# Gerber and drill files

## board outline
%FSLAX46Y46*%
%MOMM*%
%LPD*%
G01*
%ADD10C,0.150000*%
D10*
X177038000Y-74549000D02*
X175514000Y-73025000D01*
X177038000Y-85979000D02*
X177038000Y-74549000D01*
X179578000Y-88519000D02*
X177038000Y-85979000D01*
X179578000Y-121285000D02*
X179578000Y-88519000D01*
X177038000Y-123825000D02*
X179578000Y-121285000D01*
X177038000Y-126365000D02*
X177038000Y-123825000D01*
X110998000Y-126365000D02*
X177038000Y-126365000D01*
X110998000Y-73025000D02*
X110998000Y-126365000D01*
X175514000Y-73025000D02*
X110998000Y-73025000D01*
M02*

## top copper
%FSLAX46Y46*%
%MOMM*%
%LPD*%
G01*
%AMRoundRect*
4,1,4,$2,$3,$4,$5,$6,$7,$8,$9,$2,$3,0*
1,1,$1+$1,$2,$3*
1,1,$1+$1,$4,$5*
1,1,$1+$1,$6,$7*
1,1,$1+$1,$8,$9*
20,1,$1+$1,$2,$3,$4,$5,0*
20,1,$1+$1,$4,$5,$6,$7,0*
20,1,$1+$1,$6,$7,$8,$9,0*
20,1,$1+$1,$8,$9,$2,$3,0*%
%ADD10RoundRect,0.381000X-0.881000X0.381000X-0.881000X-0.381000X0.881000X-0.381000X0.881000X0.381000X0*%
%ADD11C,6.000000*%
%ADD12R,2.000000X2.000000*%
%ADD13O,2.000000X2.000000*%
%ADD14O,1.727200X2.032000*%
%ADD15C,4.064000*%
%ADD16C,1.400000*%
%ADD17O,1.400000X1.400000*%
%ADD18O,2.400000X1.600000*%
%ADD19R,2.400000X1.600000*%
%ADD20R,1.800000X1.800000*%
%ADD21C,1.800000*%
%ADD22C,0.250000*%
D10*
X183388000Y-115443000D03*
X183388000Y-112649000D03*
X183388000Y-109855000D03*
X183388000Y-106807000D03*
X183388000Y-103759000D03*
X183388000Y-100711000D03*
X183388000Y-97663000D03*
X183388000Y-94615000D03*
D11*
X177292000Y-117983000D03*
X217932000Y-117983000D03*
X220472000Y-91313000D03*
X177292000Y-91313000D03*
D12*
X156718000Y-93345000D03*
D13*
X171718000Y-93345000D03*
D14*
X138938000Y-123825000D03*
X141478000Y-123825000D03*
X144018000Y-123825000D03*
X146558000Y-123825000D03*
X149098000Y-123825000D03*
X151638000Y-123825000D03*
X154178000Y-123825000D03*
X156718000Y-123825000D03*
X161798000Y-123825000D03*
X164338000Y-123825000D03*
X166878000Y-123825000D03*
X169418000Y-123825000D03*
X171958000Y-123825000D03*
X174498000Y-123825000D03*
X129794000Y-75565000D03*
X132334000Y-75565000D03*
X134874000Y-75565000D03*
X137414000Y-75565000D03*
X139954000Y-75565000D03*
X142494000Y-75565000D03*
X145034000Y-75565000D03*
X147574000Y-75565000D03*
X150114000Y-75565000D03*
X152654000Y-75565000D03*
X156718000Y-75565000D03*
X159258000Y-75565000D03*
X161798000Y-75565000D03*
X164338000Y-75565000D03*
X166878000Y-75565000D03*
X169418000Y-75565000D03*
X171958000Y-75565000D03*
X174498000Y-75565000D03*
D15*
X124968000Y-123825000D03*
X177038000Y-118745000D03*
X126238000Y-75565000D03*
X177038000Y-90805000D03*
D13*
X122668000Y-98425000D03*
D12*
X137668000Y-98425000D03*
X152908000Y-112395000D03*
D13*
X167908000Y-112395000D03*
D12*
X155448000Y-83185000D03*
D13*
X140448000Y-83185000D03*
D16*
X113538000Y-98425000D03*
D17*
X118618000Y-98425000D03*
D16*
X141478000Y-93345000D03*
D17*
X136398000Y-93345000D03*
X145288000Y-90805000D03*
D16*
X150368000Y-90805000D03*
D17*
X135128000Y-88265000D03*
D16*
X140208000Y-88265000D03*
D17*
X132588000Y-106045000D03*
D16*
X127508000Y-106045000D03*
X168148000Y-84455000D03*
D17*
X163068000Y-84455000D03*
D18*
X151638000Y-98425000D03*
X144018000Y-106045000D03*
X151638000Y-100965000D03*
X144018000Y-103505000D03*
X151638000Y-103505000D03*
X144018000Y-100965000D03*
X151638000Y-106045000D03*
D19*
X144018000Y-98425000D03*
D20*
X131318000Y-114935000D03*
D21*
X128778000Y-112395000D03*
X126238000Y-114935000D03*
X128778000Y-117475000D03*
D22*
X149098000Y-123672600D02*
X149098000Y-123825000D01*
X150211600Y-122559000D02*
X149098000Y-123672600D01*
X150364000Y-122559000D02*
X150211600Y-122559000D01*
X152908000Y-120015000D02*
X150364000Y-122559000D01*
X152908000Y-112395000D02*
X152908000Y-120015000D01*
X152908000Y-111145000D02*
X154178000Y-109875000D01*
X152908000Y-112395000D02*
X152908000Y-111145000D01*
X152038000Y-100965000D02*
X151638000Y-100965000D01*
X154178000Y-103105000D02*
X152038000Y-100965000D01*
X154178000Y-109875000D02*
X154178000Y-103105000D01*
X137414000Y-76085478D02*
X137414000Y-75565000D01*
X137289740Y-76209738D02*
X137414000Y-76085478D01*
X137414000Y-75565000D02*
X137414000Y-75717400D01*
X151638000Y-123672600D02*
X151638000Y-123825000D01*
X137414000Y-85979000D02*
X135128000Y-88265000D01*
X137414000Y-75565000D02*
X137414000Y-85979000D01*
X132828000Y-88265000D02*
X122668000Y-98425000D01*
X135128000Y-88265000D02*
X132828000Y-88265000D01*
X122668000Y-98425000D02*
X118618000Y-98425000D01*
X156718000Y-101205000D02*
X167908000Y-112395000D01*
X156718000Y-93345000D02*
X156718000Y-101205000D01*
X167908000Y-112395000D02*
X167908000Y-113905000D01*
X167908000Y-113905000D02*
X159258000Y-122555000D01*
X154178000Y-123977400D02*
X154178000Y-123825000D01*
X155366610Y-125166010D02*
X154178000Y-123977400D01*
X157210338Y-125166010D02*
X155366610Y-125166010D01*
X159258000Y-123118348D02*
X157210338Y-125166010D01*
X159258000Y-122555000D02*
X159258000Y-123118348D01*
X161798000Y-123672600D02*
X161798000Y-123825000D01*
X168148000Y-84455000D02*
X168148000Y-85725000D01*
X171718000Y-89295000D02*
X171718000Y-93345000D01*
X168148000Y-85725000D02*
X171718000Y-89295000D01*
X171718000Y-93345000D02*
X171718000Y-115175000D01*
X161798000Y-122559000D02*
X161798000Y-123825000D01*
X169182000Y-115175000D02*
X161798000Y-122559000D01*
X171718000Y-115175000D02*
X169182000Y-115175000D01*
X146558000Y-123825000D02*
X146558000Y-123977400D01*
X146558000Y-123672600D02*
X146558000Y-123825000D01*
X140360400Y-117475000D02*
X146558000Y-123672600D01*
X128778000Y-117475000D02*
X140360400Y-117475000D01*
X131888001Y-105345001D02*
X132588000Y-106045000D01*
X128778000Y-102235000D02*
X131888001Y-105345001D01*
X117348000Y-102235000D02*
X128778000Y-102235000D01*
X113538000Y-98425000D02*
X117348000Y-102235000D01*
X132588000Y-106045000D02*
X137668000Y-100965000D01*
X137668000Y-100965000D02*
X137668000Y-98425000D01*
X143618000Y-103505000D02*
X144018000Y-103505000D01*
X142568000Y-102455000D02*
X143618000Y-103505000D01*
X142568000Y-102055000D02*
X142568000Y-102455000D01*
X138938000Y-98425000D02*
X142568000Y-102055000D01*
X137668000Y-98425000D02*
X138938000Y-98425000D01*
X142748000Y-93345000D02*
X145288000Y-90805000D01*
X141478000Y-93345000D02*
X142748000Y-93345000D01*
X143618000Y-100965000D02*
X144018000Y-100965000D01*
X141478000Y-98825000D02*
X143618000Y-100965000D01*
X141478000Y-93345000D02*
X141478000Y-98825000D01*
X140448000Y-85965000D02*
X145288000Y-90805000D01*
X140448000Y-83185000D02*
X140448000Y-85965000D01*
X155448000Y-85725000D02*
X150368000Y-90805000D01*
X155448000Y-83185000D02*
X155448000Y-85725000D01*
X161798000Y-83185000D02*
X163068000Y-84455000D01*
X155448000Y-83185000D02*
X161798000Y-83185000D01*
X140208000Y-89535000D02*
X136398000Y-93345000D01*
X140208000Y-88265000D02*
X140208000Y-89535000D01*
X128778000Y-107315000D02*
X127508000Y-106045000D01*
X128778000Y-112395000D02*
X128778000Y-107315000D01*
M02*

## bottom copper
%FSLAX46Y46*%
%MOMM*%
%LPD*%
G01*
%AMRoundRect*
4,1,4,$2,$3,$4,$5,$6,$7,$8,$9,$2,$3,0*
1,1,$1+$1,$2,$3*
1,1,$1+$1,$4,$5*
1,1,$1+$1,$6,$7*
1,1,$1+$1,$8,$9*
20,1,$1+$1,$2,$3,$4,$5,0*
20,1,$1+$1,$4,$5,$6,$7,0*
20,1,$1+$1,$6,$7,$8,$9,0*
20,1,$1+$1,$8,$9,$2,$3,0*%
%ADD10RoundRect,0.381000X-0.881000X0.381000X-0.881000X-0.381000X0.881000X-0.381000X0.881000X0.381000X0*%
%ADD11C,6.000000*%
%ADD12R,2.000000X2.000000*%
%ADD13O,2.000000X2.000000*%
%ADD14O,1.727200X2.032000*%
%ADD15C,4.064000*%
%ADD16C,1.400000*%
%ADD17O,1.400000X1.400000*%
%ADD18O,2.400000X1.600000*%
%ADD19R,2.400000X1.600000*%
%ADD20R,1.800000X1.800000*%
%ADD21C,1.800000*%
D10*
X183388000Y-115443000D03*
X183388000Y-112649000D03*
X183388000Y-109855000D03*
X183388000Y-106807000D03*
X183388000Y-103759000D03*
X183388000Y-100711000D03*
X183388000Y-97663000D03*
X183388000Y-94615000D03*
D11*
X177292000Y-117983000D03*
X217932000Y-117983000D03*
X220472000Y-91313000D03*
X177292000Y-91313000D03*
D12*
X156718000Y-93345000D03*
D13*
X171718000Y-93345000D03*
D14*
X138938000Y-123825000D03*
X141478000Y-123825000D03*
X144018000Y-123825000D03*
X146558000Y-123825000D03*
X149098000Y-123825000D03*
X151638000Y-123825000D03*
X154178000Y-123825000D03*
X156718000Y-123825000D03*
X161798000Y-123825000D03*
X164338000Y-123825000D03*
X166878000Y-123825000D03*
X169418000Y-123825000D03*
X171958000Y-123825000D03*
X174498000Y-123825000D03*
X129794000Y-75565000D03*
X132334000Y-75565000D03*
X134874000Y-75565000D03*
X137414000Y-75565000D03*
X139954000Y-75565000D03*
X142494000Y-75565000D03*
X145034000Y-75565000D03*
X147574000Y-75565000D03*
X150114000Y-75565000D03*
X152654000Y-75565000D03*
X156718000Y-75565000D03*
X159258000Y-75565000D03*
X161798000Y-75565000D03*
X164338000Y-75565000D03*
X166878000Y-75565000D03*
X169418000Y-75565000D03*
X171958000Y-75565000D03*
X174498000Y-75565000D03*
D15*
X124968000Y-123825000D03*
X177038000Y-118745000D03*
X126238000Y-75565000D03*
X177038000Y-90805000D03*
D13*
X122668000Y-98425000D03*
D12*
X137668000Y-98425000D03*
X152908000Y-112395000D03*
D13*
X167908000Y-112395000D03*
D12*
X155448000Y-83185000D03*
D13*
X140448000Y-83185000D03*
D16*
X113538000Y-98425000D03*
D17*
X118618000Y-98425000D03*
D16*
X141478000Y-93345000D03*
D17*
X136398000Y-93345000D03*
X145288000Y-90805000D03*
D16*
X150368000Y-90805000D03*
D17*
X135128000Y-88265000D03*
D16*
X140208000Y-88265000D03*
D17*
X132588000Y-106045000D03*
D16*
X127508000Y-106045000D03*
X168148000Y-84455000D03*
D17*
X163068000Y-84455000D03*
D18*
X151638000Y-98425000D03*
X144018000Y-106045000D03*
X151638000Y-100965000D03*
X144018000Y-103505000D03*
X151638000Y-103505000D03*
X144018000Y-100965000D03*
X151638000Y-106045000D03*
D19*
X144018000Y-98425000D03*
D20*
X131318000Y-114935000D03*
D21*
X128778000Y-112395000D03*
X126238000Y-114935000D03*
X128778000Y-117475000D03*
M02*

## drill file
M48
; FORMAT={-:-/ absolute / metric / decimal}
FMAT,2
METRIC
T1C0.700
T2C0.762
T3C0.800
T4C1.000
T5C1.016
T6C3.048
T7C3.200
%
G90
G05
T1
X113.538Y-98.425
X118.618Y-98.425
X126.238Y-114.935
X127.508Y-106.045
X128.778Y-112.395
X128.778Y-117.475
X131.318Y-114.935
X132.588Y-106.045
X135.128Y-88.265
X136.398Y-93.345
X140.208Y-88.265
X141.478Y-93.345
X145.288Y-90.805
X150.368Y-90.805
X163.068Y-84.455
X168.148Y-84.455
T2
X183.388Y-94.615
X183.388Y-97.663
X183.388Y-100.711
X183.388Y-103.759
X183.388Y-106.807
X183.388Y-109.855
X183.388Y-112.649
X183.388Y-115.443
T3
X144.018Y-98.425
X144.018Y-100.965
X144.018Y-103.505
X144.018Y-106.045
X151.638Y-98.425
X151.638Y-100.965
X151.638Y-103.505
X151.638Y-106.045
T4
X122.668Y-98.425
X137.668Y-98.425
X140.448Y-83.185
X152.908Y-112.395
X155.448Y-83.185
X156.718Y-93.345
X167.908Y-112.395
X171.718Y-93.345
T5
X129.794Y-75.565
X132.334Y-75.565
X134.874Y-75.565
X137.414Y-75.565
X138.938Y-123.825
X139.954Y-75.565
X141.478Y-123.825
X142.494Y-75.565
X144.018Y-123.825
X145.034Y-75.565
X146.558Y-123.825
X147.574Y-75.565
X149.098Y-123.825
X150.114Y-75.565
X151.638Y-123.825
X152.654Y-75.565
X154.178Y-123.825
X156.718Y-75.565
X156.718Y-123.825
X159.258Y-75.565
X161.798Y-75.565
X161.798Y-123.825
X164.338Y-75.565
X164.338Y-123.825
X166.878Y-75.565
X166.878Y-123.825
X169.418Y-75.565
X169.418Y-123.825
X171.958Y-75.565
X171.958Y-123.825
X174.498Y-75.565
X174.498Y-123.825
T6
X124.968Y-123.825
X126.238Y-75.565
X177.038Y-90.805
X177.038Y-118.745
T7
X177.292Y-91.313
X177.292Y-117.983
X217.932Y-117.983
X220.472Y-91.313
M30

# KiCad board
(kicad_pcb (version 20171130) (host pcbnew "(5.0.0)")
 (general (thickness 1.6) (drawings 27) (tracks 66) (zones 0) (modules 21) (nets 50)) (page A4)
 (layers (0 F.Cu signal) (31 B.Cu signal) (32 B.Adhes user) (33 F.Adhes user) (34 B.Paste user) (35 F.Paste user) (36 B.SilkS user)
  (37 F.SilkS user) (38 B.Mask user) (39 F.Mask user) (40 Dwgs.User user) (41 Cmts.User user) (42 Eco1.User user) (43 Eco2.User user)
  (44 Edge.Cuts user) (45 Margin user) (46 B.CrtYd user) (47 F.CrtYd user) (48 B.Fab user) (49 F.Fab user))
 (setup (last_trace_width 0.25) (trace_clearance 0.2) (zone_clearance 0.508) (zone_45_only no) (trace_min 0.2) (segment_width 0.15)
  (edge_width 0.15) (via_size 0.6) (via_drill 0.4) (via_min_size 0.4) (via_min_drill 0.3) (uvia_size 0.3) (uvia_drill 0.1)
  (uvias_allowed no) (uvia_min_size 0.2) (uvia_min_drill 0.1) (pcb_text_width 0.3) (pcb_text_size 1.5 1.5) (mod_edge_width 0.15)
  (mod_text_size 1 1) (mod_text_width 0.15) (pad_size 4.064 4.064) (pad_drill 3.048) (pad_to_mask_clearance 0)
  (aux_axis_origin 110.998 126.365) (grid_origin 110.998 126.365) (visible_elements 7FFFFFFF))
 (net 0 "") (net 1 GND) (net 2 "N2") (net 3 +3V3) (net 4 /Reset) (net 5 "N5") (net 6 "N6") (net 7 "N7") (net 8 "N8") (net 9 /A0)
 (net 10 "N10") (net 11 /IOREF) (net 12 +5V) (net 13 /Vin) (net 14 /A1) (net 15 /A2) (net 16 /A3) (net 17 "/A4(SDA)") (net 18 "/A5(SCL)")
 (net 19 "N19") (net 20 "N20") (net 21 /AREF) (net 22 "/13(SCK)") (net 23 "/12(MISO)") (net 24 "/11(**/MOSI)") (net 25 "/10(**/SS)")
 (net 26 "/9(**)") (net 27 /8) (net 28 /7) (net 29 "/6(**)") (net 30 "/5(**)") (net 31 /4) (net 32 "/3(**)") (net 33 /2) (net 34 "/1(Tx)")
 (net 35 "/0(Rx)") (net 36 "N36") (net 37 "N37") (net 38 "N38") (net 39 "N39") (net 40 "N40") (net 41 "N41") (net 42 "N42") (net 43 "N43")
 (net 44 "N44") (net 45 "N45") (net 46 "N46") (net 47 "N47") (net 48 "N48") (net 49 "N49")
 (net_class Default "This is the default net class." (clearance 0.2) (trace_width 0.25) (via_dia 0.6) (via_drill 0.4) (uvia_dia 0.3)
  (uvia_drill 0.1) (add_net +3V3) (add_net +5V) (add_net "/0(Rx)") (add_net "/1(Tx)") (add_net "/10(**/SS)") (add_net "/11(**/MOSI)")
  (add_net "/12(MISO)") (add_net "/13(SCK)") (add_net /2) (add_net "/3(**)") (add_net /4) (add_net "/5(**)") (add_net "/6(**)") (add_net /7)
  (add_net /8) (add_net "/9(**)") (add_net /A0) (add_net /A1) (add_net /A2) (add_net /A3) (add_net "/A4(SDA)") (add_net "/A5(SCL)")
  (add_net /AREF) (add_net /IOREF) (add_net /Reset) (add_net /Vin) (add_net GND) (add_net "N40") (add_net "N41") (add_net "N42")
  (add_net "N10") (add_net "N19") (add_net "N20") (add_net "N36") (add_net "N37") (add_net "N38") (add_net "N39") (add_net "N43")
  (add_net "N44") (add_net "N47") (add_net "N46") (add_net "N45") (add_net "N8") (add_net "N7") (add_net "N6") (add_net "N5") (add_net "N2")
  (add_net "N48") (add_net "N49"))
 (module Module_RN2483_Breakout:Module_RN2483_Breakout (layer F.Cu) (at 183.388 94.615 270)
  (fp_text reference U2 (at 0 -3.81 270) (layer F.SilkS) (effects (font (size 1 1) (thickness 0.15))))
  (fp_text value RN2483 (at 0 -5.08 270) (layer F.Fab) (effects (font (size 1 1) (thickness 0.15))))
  (pad 8 thru_hole roundrect (at 20.828 0 270) (size 1.524 2.524) (drill 0.762) (layers *.Cu *.Mask) (roundrect_rratio 0.25) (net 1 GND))
  (pad 7 thru_hole roundrect (at 18.034 0 270) (size 1.524 2.524) (drill 0.762) (layers *.Cu *.Mask) (roundrect_rratio 0.25) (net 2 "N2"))
  (pad 6 thru_hole roundrect (at 15.24 0 270) (size 1.524 2.524) (drill 0.762) (layers *.Cu *.Mask) (roundrect_rratio 0.25) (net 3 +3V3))
  (pad 5 thru_hole roundrect (at 12.192 0 270) (size 1.524 2.524) (drill 0.762) (layers *.Cu *.Mask) (roundrect_rratio 0.25) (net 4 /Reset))
  (pad 4 thru_hole roundrect (at 9.144 0 270) (size 1.524 2.524) (drill 0.762) (layers *.Cu *.Mask) (roundrect_rratio 0.25) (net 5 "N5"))
  (pad 3 thru_hole roundrect (at 6.096 0 270) (size 1.524 2.524) (drill 0.762) (layers *.Cu *.Mask) (roundrect_rratio 0.25) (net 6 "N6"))
  (pad 2 thru_hole roundrect (at 3.048 0 270) (size 1.524 2.524) (drill 0.762) (layers *.Cu *.Mask) (roundrect_rratio 0.25) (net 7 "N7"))
  (pad 1 thru_hole roundrect (at 0 0 270) (size 1.524 2.524) (drill 0.762) (layers *.Cu *.Mask) (roundrect_rratio 0.25) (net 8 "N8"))
  (pad "" thru_hole circle (at 23.368 6.096 270) (size 6 6) (drill 3.2) (layers *.Cu *.Mask))
  (pad "" thru_hole circle (at 23.368 -34.544 270) (size 6 6) (drill 3.2) (layers *.Cu *.Mask))
  (pad "" thru_hole circle (at -3.302 -37.084 270) (size 6 6) (drill 3.2) (layers *.Cu *.Mask))
  (pad "" thru_hole circle (at -3.302 6.096 270) (size 6 6) (drill 3.2) (layers *.Cu *.Mask)))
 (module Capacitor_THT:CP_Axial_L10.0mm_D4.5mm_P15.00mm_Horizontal (layer F.Cu) (at 156.718 93.345)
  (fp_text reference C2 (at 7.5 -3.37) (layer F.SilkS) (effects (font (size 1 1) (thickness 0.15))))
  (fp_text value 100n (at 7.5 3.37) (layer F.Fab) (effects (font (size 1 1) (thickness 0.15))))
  (pad 1 thru_hole rect (at 0 0) (size 2 2) (drill 1) (layers *.Cu *.Mask) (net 1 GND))
  (pad 2 thru_hole oval (at 15 0) (size 2 2) (drill 1) (layers *.Cu *.Mask) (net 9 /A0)))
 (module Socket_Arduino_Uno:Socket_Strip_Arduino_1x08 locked (layer F.Cu) (at 138.938 123.825)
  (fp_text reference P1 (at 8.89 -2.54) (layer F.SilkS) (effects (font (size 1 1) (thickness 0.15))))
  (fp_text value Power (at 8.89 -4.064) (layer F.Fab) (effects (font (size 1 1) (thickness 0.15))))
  (pad 1 thru_hole oval (at 0 0) (size 1.7272 2.032) (drill 1.016) (layers *.Cu *.Mask F.SilkS) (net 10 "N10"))
  (pad 2 thru_hole oval (at 2.54 0) (size 1.7272 2.032) (drill 1.016) (layers *.Cu *.Mask F.SilkS) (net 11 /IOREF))
  (pad 3 thru_hole oval (at 5.08 0) (size 1.7272 2.032) (drill 1.016) (layers *.Cu *.Mask F.SilkS) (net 4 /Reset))
  (pad 4 thru_hole oval (at 7.62 0) (size 1.7272 2.032) (drill 1.016) (layers *.Cu *.Mask F.SilkS) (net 3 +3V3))
  (pad 5 thru_hole oval (at 10.16 0) (size 1.7272 2.032) (drill 1.016) (layers *.Cu *.Mask F.SilkS) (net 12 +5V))
  (pad 6 thru_hole oval (at 12.7 0) (size 1.7272 2.032) (drill 1.016) (layers *.Cu *.Mask F.SilkS) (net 1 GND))
  (pad 7 thru_hole oval (at 15.24 0) (size 1.7272 2.032) (drill 1.016) (layers *.Cu *.Mask F.SilkS) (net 1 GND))
  (pad 8 thru_hole oval (at 17.78 0) (size 1.7272 2.032) (drill 1.016) (layers *.Cu *.Mask F.SilkS) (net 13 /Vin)))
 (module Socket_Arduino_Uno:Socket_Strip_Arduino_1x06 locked (layer F.Cu) (at 161.798 123.825)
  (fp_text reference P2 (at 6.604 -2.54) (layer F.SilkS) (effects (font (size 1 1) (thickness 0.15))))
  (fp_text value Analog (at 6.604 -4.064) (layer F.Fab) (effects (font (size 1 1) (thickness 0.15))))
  (pad 1 thru_hole oval (at 0 0) (size 1.7272 2.032) (drill 1.016) (layers *.Cu *.Mask F.SilkS) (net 9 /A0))
  (pad 2 thru_hole oval (at 2.54 0) (size 1.7272 2.032) (drill 1.016) (layers *.Cu *.Mask F.SilkS) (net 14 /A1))
  (pad 3 thru_hole oval (at 5.08 0) (size 1.7272 2.032) (drill 1.016) (layers *.Cu *.Mask F.SilkS) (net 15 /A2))
  (pad 4 thru_hole oval (at 7.62 0) (size 1.7272 2.032) (drill 1.016) (layers *.Cu *.Mask F.SilkS) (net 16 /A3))
  (pad 5 thru_hole oval (at 10.16 0) (size 1.7272 2.032) (drill 1.016) (layers *.Cu *.Mask F.SilkS) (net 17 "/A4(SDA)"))
  (pad 6 thru_hole oval (at 12.7 0) (size 1.7272 2.032) (drill 1.016) (layers *.Cu *.Mask F.SilkS) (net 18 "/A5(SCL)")))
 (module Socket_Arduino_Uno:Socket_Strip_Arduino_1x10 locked (layer F.Cu) (at 129.794 75.565)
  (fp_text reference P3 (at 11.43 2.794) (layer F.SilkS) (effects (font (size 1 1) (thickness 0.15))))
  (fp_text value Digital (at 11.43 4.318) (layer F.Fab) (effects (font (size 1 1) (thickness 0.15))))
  (pad 1 thru_hole oval (at 0 0) (size 1.7272 2.032) (drill 1.016) (layers *.Cu *.Mask F.SilkS) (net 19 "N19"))
  (pad 2 thru_hole oval (at 2.54 0) (size 1.7272 2.032) (drill 1.016) (layers *.Cu *.Mask F.SilkS) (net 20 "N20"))
  (pad 3 thru_hole oval (at 5.08 0) (size 1.7272 2.032) (drill 1.016) (layers *.Cu *.Mask F.SilkS) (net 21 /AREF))
  (pad 4 thru_hole oval (at 7.62 0) (size 1.7272 2.032) (drill 1.016) (layers *.Cu *.Mask F.SilkS) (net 1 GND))
  (pad 5 thru_hole oval (at 10.16 0) (size 1.7272 2.032) (drill 1.016) (layers *.Cu *.Mask F.SilkS) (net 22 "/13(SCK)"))
  (pad 6 thru_hole oval (at 12.7 0) (size 1.7272 2.032) (drill 1.016) (layers *.Cu *.Mask F.SilkS) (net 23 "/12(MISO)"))
  (pad 7 thru_hole oval (at 15.24 0) (size 1.7272 2.032) (drill 1.016) (layers *.Cu *.Mask F.SilkS) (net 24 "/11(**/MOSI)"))
  (pad 8 thru_hole oval (at 17.78 0) (size 1.7272 2.032) (drill 1.016) (layers *.Cu *.Mask F.SilkS) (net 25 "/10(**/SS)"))
  (pad 9 thru_hole oval (at 20.32 0) (size 1.7272 2.032) (drill 1.016) (layers *.Cu *.Mask F.SilkS) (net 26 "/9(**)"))
  (pad 10 thru_hole oval (at 22.86 0) (size 1.7272 2.032) (drill 1.016) (layers *.Cu *.Mask F.SilkS) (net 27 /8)))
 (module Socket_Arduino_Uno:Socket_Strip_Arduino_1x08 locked (layer F.Cu) (at 156.718 75.565)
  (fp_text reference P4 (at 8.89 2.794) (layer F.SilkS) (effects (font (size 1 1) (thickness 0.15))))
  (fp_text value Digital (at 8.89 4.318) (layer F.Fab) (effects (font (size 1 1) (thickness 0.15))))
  (pad 1 thru_hole oval (at 0 0) (size 1.7272 2.032) (drill 1.016) (layers *.Cu *.Mask F.SilkS) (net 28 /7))
  (pad 2 thru_hole oval (at 2.54 0) (size 1.7272 2.032) (drill 1.016) (layers *.Cu *.Mask F.SilkS) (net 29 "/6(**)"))
  (pad 3 thru_hole oval (at 5.08 0) (size 1.7272 2.032) (drill 1.016) (layers *.Cu *.Mask F.SilkS) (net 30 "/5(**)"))
  (pad 4 thru_hole oval (at 7.62 0) (size 1.7272 2.032) (drill 1.016) (layers *.Cu *.Mask F.SilkS) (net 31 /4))
  (pad 5 thru_hole oval (at 10.16 0) (size 1.7272 2.032) (drill 1.016) (layers *.Cu *.Mask F.SilkS) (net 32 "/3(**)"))
  (pad 6 thru_hole oval (at 12.7 0) (size 1.7272 2.032) (drill 1.016) (layers *.Cu *.Mask F.SilkS) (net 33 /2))
  (pad 7 thru_hole oval (at 15.24 0) (size 1.7272 2.032) (drill 1.016) (layers *.Cu *.Mask F.SilkS) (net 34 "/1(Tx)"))
  (pad 8 thru_hole oval (at 17.78 0) (size 1.7272 2.032) (drill 1.016) (layers *.Cu *.Mask F.SilkS) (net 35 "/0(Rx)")))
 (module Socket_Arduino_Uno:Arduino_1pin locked (layer F.Cu) (at 124.968 123.825)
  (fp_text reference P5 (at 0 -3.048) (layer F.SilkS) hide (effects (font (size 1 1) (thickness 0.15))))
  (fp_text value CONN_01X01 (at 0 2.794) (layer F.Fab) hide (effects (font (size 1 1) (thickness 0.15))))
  (pad 1 thru_hole circle (at 0 0) (size 4.064 4.064) (drill 3.048) (layers *.Cu *.Mask F.SilkS) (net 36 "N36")))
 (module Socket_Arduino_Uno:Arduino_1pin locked (layer F.Cu) (at 177.038 118.745)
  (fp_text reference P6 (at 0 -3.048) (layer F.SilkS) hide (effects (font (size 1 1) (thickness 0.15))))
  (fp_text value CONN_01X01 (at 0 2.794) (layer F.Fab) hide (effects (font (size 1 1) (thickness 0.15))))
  (pad 1 thru_hole circle (at 0 0) (size 4.064 4.064) (drill 3.048) (layers *.Cu *.Mask F.SilkS) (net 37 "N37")))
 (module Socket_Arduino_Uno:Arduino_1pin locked (layer F.Cu) (at 126.238 75.565)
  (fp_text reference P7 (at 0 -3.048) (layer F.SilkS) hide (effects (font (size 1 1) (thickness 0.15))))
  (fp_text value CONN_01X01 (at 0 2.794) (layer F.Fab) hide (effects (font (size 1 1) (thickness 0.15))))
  (pad 1 thru_hole circle (at 0 0) (size 4.064 4.064) (drill 3.048) (layers *.Cu *.Mask F.SilkS) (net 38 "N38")))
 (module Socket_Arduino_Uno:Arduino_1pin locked (layer F.Cu) (at 177.038 90.805)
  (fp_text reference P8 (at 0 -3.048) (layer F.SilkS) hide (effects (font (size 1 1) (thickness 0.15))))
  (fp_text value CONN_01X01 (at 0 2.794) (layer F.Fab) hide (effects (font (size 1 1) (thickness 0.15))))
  (pad 1 thru_hole circle (at 0 0) (size 4.064 4.064) (drill 3.048) (layers *.Cu *.Mask F.SilkS) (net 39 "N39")))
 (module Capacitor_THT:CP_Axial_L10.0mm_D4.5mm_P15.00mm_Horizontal (layer F.Cu) (at 137.668 98.425 180)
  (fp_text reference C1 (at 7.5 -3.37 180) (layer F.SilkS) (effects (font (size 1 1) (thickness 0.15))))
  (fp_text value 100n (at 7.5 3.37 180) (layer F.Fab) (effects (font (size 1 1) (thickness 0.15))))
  (pad 2 thru_hole oval (at 15 0 180) (size 2 2) (drill 1) (layers *.Cu *.Mask) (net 1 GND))
  (pad 1 thru_hole rect (at 0 0 180) (size 2 2) (drill 1) (layers *.Cu *.Mask) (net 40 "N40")))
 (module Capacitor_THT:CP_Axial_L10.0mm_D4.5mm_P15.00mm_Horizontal (layer F.Cu) (at 152.908 112.395)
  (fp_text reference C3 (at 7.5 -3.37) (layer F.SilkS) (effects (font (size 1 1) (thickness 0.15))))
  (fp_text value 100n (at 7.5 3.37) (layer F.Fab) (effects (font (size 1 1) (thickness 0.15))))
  (pad 1 thru_hole rect (at 0 0) (size 2 2) (drill 1) (layers *.Cu *.Mask) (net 12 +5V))
  (pad 2 thru_hole oval (at 15 0) (size 2 2) (drill 1) (layers *.Cu *.Mask) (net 1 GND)))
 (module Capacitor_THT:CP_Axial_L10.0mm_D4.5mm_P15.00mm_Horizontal (layer F.Cu) (at 155.448 83.185 180)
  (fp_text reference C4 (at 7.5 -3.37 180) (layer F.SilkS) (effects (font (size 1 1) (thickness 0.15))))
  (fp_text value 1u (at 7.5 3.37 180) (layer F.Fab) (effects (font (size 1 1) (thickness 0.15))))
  (pad 1 thru_hole rect (at 0 0 180) (size 2 2) (drill 1) (layers *.Cu *.Mask) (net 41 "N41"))
  (pad 2 thru_hole oval (at 15 0 180) (size 2 2) (drill 1) (layers *.Cu *.Mask) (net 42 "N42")))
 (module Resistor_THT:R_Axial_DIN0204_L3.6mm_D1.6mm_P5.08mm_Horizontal (layer F.Cu) (at 113.538 98.425)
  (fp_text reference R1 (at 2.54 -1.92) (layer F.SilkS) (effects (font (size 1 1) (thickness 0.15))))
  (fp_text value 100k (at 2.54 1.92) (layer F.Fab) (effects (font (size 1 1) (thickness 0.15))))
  (pad 1 thru_hole circle (at 0 0) (size 1.4 1.4) (drill 0.7) (layers *.Cu *.Mask) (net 40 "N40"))
  (pad 2 thru_hole oval (at 5.08 0) (size 1.4 1.4) (drill 0.7) (layers *.Cu *.Mask) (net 1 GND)))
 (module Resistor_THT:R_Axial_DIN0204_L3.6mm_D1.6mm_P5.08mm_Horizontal (layer F.Cu) (at 141.478 93.345 180)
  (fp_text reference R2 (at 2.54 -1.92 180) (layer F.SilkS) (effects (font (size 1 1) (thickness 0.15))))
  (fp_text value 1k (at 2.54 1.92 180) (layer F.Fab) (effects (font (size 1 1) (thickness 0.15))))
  (pad 1 thru_hole circle (at 0 0 180) (size 1.4 1.4) (drill 0.7) (layers *.Cu *.Mask) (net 42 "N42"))
  (pad 2 thru_hole oval (at 5.08 0 180) (size 1.4 1.4) (drill 0.7) (layers *.Cu *.Mask) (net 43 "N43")))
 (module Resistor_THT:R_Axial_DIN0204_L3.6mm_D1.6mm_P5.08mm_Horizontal (layer F.Cu) (at 150.368 90.805 180)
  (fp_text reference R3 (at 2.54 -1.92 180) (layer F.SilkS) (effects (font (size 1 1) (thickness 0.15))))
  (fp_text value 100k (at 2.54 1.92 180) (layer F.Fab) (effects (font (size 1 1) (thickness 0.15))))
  (pad 2 thru_hole oval (at 5.08 0 180) (size 1.4 1.4) (drill 0.7) (layers *.Cu *.Mask) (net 42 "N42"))
  (pad 1 thru_hole circle (at 0 0 180) (size 1.4 1.4) (drill 0.7) (layers *.Cu *.Mask) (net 41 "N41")))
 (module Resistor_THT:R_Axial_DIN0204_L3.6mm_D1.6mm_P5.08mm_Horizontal (layer F.Cu) (at 140.208 88.265 180)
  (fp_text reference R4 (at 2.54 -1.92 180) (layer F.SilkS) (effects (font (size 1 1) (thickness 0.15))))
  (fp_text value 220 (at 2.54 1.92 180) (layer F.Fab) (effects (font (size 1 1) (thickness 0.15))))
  (pad 2 thru_hole oval (at 5.08 0 180) (size 1.4 1.4) (drill 0.7) (layers *.Cu *.Mask) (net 1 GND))
  (pad 1 thru_hole circle (at 0 0 180) (size 1.4 1.4) (drill 0.7) (layers *.Cu *.Mask) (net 43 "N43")))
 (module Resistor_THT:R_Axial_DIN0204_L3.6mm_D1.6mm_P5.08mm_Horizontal (layer F.Cu) (at 127.508 106.045)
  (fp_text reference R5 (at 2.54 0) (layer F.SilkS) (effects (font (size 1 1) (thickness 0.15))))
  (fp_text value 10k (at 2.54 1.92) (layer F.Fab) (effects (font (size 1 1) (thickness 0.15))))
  (pad 2 thru_hole oval (at 5.08 0) (size 1.4 1.4) (drill 0.7) (layers *.Cu *.Mask) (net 40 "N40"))
  (pad 1 thru_hole circle (at 0 0) (size 1.4 1.4) (drill 0.7) (layers *.Cu *.Mask) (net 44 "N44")))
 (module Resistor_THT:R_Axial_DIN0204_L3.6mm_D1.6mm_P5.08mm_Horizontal (layer F.Cu) (at 168.148 84.455 180)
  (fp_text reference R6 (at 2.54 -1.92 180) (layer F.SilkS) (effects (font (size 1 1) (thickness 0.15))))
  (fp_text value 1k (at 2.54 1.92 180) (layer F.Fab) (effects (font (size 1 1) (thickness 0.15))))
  (pad 1 thru_hole circle (at 0 0 180) (size 1.4 1.4) (drill 0.7) (layers *.Cu *.Mask) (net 9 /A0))
  (pad 2 thru_hole oval (at 5.08 0 180) (size 1.4 1.4) (drill 0.7) (layers *.Cu *.Mask) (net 41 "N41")))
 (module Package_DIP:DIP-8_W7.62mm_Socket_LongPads (layer F.Cu) (at 144.018 98.425)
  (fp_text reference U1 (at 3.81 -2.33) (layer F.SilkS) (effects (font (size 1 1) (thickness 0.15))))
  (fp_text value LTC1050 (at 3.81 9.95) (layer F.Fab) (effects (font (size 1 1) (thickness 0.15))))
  (pad 8 thru_hole oval (at 7.62 0) (size 2.4 1.6) (drill 0.8) (layers *.Cu *.Mask) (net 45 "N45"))
  (pad 4 thru_hole oval (at 0 7.62) (size 2.4 1.6) (drill 0.8) (layers *.Cu *.Mask) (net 1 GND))
  (pad 7 thru_hole oval (at 7.62 2.54) (size 2.4 1.6) (drill 0.8) (layers *.Cu *.Mask) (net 12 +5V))
  (pad 3 thru_hole oval (at 0 5.08) (size 2.4 1.6) (drill 0.8) (layers *.Cu *.Mask) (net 40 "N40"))
  (pad 6 thru_hole oval (at 7.62 5.08) (size 2.4 1.6) (drill 0.8) (layers *.Cu *.Mask) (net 41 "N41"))
  (pad 2 thru_hole oval (at 0 2.54) (size 2.4 1.6) (drill 0.8) (layers *.Cu *.Mask) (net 42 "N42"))
  (pad 5 thru_hole oval (at 7.62 7.62) (size 2.4 1.6) (drill 0.8) (layers *.Cu *.Mask) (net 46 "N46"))
  (pad 1 thru_hole rect (at 0 0) (size 2.4 1.6) (drill 0.8) (layers *.Cu *.Mask) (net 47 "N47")))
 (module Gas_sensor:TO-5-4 (layer F.Cu) (at 131.318 114.935 180)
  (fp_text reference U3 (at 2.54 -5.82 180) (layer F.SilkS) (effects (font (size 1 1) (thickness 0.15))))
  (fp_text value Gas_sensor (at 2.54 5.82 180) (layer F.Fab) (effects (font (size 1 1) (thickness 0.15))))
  (pad 1 thru_hole rect (at 0 0 180) (size 1.8 1.8) (drill 0.7) (layers *.Cu *.Mask) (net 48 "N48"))
  (pad 2 thru_hole circle (at 2.54 2.54 180) (size 1.8 1.8) (drill 0.7) (layers *.Cu *.Mask) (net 44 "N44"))
  (pad 3 thru_hole circle (at 5.08 0 180) (size 1.8 1.8) (drill 0.7) (layers *.Cu *.Mask) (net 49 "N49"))
  (pad 4 thru_hole circle (at 2.54 -2.54 180) (size 1.8 1.8) (drill 0.7) (layers *.Cu *.Mask) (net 3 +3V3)))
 (gr_line (start 177.038 74.549) (end 175.514 73.025) (angle 90) (layer Edge.Cuts) (width 0.15))
 (gr_line (start 177.038 85.979) (end 177.038 74.549) (angle 90) (layer Edge.Cuts) (width 0.15))
 (gr_line (start 179.578 88.519) (end 177.038 85.979) (angle 90) (layer Edge.Cuts) (width 0.15))
 (gr_line (start 179.578 121.285) (end 179.578 88.519) (angle 90) (layer Edge.Cuts) (width 0.15))
 (gr_line (start 177.038 123.825) (end 179.578 121.285) (angle 90) (layer Edge.Cuts) (width 0.15))
 (gr_line (start 177.038 126.365) (end 177.038 123.825) (angle 90) (layer Edge.Cuts) (width 0.15))
 (gr_line (start 110.998 126.365) (end 177.038 126.365) (angle 90) (layer Edge.Cuts) (width 0.15))
 (gr_line (start 110.998 73.025) (end 110.998 126.365) (angle 90) (layer Edge.Cuts) (width 0.15))
 (gr_line (start 175.514 73.025) (end 110.998 73.025) (angle 90) (layer Edge.Cuts) (width 0.15))
 (segment (start 149.098 123.6726) (end 149.098 123.825) (width 0.25) (layer F.Cu) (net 12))
 (segment (start 150.2116 122.559) (end 149.098 123.6726) (width 0.25) (layer F.Cu) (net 12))
 (segment (start 150.364 122.559) (end 150.2116 122.559) (width 0.25) (layer F.Cu) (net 12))
 (segment (start 152.908 120.015) (end 150.364 122.559) (width 0.25) (layer F.Cu) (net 12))
 (segment (start 152.908 112.395) (end 152.908 120.015) (width 0.25) (layer F.Cu) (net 12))
 (segment (start 152.908 111.145) (end 154.178 109.875) (width 0.25) (layer F.Cu) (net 12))
 (segment (start 152.908 112.395) (end 152.908 111.145) (width 0.25) (layer F.Cu) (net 12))
 (segment (start 152.038 100.965) (end 151.638 100.965) (width 0.25) (layer F.Cu) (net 12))
 (segment (start 154.178 103.105) (end 152.038 100.965) (width 0.25) (layer F.Cu) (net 12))
 (segment (start 154.178 109.875) (end 154.178 103.105) (width 0.25) (layer F.Cu) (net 12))
 (segment (start 137.414 76.085478) (end 137.414 75.565) (width 0.25) (layer F.Cu) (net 1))
 (segment (start 137.28974 76.209738) (end 137.414 76.085478) (width 0.25) (layer F.Cu) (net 1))
 (segment (start 137.414 75.565) (end 137.414 75.7174) (width 0.25) (layer F.Cu) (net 1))
 (segment (start 151.638 123.6726) (end 151.638 123.825) (width 0.25) (layer F.Cu) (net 1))
 (segment (start 137.414 85.979) (end 135.128 88.265) (width 0.25) (layer F.Cu) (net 1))
 (segment (start 137.414 75.565) (end 137.414 85.979) (width 0.25) (layer F.Cu) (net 1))
 (segment (start 132.828 88.265) (end 122.668 98.425) (width 0.25) (layer F.Cu) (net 1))
 (segment (start 135.128 88.265) (end 132.828 88.265) (width 0.25) (layer F.Cu) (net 1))
 (segment (start 122.668 98.425) (end 118.618 98.425) (width 0.25) (layer F.Cu) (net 1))
 (segment (start 156.718 101.205) (end 167.908 112.395) (width 0.25) (layer F.Cu) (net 1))
 (segment (start 156.718 93.345) (end 156.718 101.205) (width 0.25) (layer F.Cu) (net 1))
 (segment (start 167.908 112.395) (end 167.908 113.905) (width 0.25) (layer F.Cu) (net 1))
 (segment (start 167.908 113.905) (end 159.258 122.555) (width 0.25) (layer F.Cu) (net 1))
 (segment (start 154.178 123.9774) (end 154.178 123.825) (width 0.25) (layer F.Cu) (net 1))
 (segment (start 155.36661 125.16601) (end 154.178 123.9774) (width 0.25) (layer F.Cu) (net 1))
 (segment (start 157.210338 125.16601) (end 155.36661 125.16601) (width 0.25) (layer F.Cu) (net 1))
 (segment (start 159.258 123.118348) (end 157.210338 125.16601) (width 0.25) (layer F.Cu) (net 1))
 (segment (start 159.258 122.555) (end 159.258 123.118348) (width 0.25) (layer F.Cu) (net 1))
 (segment (start 161.798 123.6726) (end 161.798 123.825) (width 0.25) (layer F.Cu) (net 9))
 (segment (start 168.148 84.455) (end 168.148 85.725) (width 0.25) (layer F.Cu) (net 9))
 (segment (start 171.718 89.295) (end 171.718 93.345) (width 0.25) (layer F.Cu) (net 9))
 (segment (start 168.148 85.725) (end 171.718 89.295) (width 0.25) (layer F.Cu) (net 9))
 (segment (start 171.718 93.345) (end 171.718 115.175) (width 0.25) (layer F.Cu) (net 9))
 (segment (start 161.798 122.559) (end 161.798 123.825) (width 0.25) (layer F.Cu) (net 9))
 (segment (start 169.182 115.175) (end 161.798 122.559) (width 0.25) (layer F.Cu) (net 9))
 (segment (start 171.718 115.175) (end 169.182 115.175) (width 0.25) (layer F.Cu) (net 9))
 (segment (start 146.558 123.825) (end 146.558 123.9774) (width 0.25) (layer F.Cu) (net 3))
 (segment (start 146.558 123.6726) (end 146.558 123.825) (width 0.25) (layer F.Cu) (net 3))
 (segment (start 140.3604 117.475) (end 146.558 123.6726) (width 0.25) (layer F.Cu) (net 3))
 (segment (start 128.778 117.475) (end 140.3604 117.475) (width 0.25) (layer F.Cu) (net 3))
 (segment (start 131.888001 105.345001) (end 132.588 106.045) (width 0.25) (layer F.Cu) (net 40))
 (segment (start 128.778 102.235) (end 131.888001 105.345001) (width 0.25) (layer F.Cu) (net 40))
 (segment (start 117.348 102.235) (end 128.778 102.235) (width 0.25) (layer F.Cu) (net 40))
 (segment (start 113.538 98.425) (end 117.348 102.235) (width 0.25) (layer F.Cu) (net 40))
 (segment (start 132.588 106.045) (end 137.668 100.965) (width 0.25) (layer F.Cu) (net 40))
 (segment (start 137.668 100.965) (end 137.668 98.425) (width 0.25) (layer F.Cu) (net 40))
 (segment (start 143.618 103.505) (end 144.018 103.505) (width 0.25) (layer F.Cu) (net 40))
 (segment (start 142.568 102.455) (end 143.618 103.505) (width 0.25) (layer F.Cu) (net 40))
 (segment (start 142.568 102.055) (end 142.568 102.455) (width 0.25) (layer F.Cu) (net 40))
 (segment (start 138.938 98.425) (end 142.568 102.055) (width 0.25) (layer F.Cu) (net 40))
 (segment (start 137.668 98.425) (end 138.938 98.425) (width 0.25) (layer F.Cu) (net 40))
 (segment (start 142.748 93.345) (end 145.288 90.805) (width 0.25) (layer F.Cu) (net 42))
 (segment (start 141.478 93.345) (end 142.748 93.345) (width 0.25) (layer F.Cu) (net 42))
 (segment (start 143.618 100.965) (end 144.018 100.965) (width 0.25) (layer F.Cu) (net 42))
 (segment (start 141.478 98.825) (end 143.618 100.965) (width 0.25) (layer F.Cu) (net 42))
 (segment (start 141.478 93.345) (end 141.478 98.825) (width 0.25) (layer F.Cu) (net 42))
 (segment (start 140.448 85.965) (end 145.288 90.805) (width 0.25) (layer F.Cu) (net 42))
 (segment (start 140.448 83.185) (end 140.448 85.965) (width 0.25) (layer F.Cu) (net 42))
 (segment (start 155.448 85.725) (end 150.368 90.805) (width 0.25) (layer F.Cu) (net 41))
 (segment (start 155.448 83.185) (end 155.448 85.725) (width 0.25) (layer F.Cu) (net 41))
 (segment (start 161.798 83.185) (end 163.068 84.455) (width 0.25) (layer F.Cu) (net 41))
 (segment (start 155.448 83.185) (end 161.798 83.185) (width 0.25) (layer F.Cu) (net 41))
 (segment (start 140.208 89.535) (end 136.398 93.345) (width 0.25) (layer F.Cu) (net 43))
 (segment (start 140.208 88.265) (end 140.208 89.535) (width 0.25) (layer F.Cu) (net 43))
 (segment (start 128.778 107.315) (end 127.508 106.045) (width 0.25) (layer F.Cu) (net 44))
 (segment (start 128.778 112.395) (end 128.778 107.315) (width 0.25) (layer F.Cu) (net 44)))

